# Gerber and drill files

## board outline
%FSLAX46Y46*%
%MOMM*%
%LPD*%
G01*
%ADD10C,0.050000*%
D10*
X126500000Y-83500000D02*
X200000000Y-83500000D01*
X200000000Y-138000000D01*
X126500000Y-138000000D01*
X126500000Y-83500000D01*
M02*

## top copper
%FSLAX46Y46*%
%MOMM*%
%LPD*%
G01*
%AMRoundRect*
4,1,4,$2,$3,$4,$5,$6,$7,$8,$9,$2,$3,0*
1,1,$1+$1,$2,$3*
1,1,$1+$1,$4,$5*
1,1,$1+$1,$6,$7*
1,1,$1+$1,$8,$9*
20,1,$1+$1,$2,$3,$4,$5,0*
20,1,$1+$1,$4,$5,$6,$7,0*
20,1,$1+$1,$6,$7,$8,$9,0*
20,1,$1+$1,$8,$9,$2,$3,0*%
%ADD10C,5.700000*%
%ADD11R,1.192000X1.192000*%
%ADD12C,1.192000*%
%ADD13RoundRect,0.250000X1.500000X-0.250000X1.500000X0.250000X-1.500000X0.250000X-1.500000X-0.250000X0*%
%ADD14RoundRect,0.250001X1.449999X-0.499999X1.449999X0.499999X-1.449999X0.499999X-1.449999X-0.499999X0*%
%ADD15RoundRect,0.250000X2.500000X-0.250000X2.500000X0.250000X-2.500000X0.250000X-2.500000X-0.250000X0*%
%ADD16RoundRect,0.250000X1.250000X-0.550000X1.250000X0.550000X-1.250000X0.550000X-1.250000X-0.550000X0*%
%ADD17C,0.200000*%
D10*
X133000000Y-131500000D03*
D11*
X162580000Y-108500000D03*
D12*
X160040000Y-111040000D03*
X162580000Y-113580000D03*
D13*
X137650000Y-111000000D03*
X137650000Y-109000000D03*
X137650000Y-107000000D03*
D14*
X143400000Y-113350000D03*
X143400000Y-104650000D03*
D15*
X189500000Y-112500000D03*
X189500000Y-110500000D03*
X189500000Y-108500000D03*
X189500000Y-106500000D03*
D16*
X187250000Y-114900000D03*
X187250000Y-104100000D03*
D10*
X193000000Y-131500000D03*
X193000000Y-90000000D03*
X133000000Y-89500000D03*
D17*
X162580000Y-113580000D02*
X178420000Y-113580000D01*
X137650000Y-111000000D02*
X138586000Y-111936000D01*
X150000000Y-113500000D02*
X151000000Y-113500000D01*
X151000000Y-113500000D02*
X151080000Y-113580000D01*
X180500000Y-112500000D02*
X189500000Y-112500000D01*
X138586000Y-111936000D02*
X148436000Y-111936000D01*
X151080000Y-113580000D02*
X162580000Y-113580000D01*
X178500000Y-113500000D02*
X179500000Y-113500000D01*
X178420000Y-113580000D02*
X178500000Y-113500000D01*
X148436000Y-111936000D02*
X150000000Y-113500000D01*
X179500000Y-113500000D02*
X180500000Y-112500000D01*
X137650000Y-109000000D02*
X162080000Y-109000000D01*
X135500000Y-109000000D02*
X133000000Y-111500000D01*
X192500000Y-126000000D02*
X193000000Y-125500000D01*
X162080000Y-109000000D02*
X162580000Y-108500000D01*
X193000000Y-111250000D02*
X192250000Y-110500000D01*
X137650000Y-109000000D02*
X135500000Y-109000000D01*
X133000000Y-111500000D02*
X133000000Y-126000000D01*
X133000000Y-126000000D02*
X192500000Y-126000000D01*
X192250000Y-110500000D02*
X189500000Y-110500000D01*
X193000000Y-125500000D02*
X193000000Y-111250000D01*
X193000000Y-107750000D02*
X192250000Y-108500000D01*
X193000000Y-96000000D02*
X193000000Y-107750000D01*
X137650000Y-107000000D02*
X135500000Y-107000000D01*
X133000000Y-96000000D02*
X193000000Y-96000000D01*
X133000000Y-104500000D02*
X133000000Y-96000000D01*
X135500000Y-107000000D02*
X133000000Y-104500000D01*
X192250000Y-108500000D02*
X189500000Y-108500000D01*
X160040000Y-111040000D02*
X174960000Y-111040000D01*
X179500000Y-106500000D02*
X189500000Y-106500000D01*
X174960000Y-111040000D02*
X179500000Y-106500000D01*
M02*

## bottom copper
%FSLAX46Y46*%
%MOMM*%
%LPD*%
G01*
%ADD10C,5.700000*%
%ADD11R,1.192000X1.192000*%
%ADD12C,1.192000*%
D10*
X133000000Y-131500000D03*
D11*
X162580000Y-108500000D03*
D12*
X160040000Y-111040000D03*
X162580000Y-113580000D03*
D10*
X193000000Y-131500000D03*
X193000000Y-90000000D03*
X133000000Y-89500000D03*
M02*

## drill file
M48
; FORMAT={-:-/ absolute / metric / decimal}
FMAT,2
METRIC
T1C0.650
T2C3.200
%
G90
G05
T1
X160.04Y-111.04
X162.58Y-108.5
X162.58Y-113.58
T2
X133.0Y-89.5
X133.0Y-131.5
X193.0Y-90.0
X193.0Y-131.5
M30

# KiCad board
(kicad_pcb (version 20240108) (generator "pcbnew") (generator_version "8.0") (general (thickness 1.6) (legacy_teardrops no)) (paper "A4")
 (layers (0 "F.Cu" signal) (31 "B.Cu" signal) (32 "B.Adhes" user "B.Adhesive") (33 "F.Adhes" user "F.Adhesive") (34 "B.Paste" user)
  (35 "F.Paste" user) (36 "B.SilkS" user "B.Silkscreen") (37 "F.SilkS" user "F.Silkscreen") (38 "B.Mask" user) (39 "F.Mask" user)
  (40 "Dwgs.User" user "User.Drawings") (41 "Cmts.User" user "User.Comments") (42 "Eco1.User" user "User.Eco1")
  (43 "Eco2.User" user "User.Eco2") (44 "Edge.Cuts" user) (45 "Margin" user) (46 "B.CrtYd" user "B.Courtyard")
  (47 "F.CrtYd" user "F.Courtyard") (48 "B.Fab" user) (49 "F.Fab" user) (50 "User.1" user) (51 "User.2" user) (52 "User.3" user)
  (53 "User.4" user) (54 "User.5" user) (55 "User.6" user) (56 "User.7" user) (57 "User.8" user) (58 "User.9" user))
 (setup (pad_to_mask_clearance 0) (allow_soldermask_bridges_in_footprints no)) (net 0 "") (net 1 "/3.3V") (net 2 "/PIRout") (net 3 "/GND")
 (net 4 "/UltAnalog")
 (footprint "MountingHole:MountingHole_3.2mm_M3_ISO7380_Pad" (layer "F.Cu") (at 133 131.5)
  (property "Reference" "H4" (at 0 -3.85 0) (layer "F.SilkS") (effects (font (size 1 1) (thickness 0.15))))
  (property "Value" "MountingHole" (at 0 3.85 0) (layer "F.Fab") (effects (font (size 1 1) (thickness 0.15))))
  (pad "1" thru_hole circle (at 0 0) (size 5.7 5.7) (drill 3.2) (layers "*.Cu" "*.Mask") (remove_unused_layers no)))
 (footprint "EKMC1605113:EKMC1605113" (layer "F.Cu") (at 162.58 108.5 90)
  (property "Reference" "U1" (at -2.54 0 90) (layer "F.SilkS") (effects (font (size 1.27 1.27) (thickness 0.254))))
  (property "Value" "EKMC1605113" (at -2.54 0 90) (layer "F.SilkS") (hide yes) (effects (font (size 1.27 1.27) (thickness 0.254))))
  (pad "1" thru_hole rect (at 0 0 90) (size 1.192 1.192) (drill 0.65) (layers "*.Cu" "*.Mask") (remove_unused_layers no) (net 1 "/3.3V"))
  (pad "2" thru_hole circle (at -2.54 -2.54 90) (size 1.192 1.192) (drill 0.65) (layers "*.Cu" "*.Mask") (remove_unused_layers no)
   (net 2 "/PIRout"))
  (pad "3" thru_hole circle (at -5.08 0 90) (size 1.192 1.192) (drill 0.65) (layers "*.Cu" "*.Mask") (remove_unused_layers no)
   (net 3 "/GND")))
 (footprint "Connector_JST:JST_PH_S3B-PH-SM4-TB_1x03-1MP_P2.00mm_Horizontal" (layer "F.Cu") (at 140.5 109 90)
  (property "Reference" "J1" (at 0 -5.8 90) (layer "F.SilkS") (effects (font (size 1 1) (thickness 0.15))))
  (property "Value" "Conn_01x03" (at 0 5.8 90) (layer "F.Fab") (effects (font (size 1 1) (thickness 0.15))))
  (pad "1" smd roundrect (at -2 -2.85 90) (size 1 3.5) (layers "F.Cu" "F.Paste" "F.Mask") (roundrect_rratio 0.25) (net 3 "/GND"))
  (pad "2" smd roundrect (at 0 -2.85 90) (size 1 3.5) (layers "F.Cu" "F.Paste" "F.Mask") (roundrect_rratio 0.25) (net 1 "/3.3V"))
  (pad "3" smd roundrect (at 2 -2.85 90) (size 1 3.5) (layers "F.Cu" "F.Paste" "F.Mask") (roundrect_rratio 0.25) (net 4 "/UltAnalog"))
  (pad "MP" smd roundrect (at -4.35 2.9 90) (size 1.5 3.4) (layers "F.Cu" "F.Paste" "F.Mask") (roundrect_rratio 0.166667))
  (pad "MP" smd roundrect (at 4.35 2.9 90) (size 1.5 3.4) (layers "F.Cu" "F.Paste" "F.Mask") (roundrect_rratio 0.166667)))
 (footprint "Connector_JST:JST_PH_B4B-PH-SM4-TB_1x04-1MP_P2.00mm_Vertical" (layer "F.Cu") (at 189 109.5 90)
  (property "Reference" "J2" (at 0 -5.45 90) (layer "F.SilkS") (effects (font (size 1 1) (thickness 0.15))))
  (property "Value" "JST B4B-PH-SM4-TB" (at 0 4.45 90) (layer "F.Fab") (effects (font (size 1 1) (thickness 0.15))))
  (pad "1" smd roundrect (at -3 0.5 90) (size 1 5.5) (layers "F.Cu" "F.Paste" "F.Mask") (roundrect_rratio 0.25) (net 3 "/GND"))
  (pad "2" smd roundrect (at -1 0.5 90) (size 1 5.5) (layers "F.Cu" "F.Paste" "F.Mask") (roundrect_rratio 0.25) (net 1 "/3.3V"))
  (pad "3" smd roundrect (at 1 0.5 90) (size 1 5.5) (layers "F.Cu" "F.Paste" "F.Mask") (roundrect_rratio 0.25) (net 4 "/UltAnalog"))
  (pad "4" smd roundrect (at 3 0.5 90) (size 1 5.5) (layers "F.Cu" "F.Paste" "F.Mask") (roundrect_rratio 0.25) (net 2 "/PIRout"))
  (pad "MP" smd roundrect (at -5.4 -1.75 90) (size 1.6 3) (layers "F.Cu" "F.Paste" "F.Mask") (roundrect_rratio 0.15625))
  (pad "MP" smd roundrect (at 5.4 -1.75 90) (size 1.6 3) (layers "F.Cu" "F.Paste" "F.Mask") (roundrect_rratio 0.15625)))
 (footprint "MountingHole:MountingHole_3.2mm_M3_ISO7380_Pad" (layer "F.Cu") (at 193 131.5)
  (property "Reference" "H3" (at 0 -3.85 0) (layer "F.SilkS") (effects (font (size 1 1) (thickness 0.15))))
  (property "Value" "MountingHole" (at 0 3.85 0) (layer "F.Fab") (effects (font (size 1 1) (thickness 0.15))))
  (pad "1" thru_hole circle (at 0 0) (size 5.7 5.7) (drill 3.2) (layers "*.Cu" "*.Mask") (remove_unused_layers no)))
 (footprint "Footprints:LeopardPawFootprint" (layer "F.Cu") (at 170.5 88)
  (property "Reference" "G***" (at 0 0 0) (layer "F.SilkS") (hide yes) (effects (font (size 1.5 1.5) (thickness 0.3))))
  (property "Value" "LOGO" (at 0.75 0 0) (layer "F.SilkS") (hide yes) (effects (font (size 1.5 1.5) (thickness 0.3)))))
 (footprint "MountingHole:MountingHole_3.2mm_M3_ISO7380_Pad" (layer "F.Cu") (at 193 90)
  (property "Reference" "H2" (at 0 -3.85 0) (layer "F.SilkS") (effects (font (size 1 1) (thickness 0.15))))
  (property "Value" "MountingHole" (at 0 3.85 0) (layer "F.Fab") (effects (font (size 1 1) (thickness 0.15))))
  (pad "1" thru_hole circle (at 0 0) (size 5.7 5.7) (drill 3.2) (layers "*.Cu" "*.Mask") (remove_unused_layers no)))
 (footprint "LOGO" (layer "F.Cu") (at 161.5 88)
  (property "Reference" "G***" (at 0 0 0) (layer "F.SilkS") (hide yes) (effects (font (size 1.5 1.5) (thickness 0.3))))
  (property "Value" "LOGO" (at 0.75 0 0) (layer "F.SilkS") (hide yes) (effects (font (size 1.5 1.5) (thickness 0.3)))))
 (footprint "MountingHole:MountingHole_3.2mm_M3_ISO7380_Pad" (layer "F.Cu") (at 133 89.5)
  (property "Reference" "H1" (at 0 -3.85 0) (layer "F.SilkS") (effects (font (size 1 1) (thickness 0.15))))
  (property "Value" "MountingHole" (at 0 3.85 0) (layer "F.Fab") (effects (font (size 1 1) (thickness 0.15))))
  (pad "1" thru_hole circle (at 0 0) (size 5.7 5.7) (drill 3.2) (layers "*.Cu" "*.Mask") (remove_unused_layers no)))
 (gr_rect (start 126.5 83.5) (end 200 138) (stroke (width 0.05) (type default)) (fill none) (layer "Edge.Cuts"))
 (segment (start 162.58 113.58) (end 178.42 113.58) (width 0.2) (layer "F.Cu") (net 3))
 (segment (start 137.65 111) (end 138.586 111.936) (width 0.2) (layer "F.Cu") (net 3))
 (segment (start 150 113.5) (end 151 113.5) (width 0.2) (layer "F.Cu") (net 3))
 (segment (start 151 113.5) (end 151.08 113.58) (width 0.2) (layer "F.Cu") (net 3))
 (segment (start 180.5 112.5) (end 189.5 112.5) (width 0.2) (layer "F.Cu") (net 3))
 (segment (start 138.586 111.936) (end 148.436 111.936) (width 0.2) (layer "F.Cu") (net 3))
 (segment (start 151.08 113.58) (end 162.58 113.58) (width 0.2) (layer "F.Cu") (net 3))
 (segment (start 178.5 113.5) (end 179.5 113.5) (width 0.2) (layer "F.Cu") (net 3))
 (segment (start 178.42 113.58) (end 178.5 113.5) (width 0.2) (layer "F.Cu") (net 3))
 (segment (start 148.436 111.936) (end 150 113.5) (width 0.2) (layer "F.Cu") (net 3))
 (segment (start 179.5 113.5) (end 180.5 112.5) (width 0.2) (layer "F.Cu") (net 3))
 (segment (start 137.65 109) (end 162.08 109) (width 0.2) (layer "F.Cu") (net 1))
 (segment (start 135.5 109) (end 133 111.5) (width 0.2) (layer "F.Cu") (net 1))
 (segment (start 192.5 126) (end 193 125.5) (width 0.2) (layer "F.Cu") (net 1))
 (segment (start 162.08 109) (end 162.58 108.5) (width 0.2) (layer "F.Cu") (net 1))
 (segment (start 193 111.25) (end 192.25 110.5) (width 0.2) (layer "F.Cu") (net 1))
 (segment (start 137.65 109) (end 135.5 109) (width 0.2) (layer "F.Cu") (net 1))
 (segment (start 133 111.5) (end 133 126) (width 0.2) (layer "F.Cu") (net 1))
 (segment (start 133 126) (end 192.5 126) (width 0.2) (layer "F.Cu") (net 1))
 (segment (start 192.25 110.5) (end 189.5 110.5) (width 0.2) (layer "F.Cu") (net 1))
 (segment (start 193 125.5) (end 193 111.25) (width 0.2) (layer "F.Cu") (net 1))
 (segment (start 193 107.75) (end 192.25 108.5) (width 0.2) (layer "F.Cu") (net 4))
 (segment (start 193 96) (end 193 107.75) (width 0.2) (layer "F.Cu") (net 4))
 (segment (start 137.65 107) (end 135.5 107) (width 0.2) (layer "F.Cu") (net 4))
 (segment (start 133 96) (end 193 96) (width 0.2) (layer "F.Cu") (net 4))
 (segment (start 133 104.5) (end 133 96) (width 0.2) (layer "F.Cu") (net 4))
 (segment (start 135.5 107) (end 133 104.5) (width 0.2) (layer "F.Cu") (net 4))
 (segment (start 192.25 108.5) (end 189.5 108.5) (width 0.2) (layer "F.Cu") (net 4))
 (segment (start 160.04 111.04) (end 174.96 111.04) (width 0.2) (layer "F.Cu") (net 2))
 (segment (start 179.5 106.5) (end 189.5 106.5) (width 0.2) (layer "F.Cu") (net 2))
 (segment (start 174.96 111.04) (end 179.5 106.5) (width 0.2) (layer "F.Cu") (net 2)))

